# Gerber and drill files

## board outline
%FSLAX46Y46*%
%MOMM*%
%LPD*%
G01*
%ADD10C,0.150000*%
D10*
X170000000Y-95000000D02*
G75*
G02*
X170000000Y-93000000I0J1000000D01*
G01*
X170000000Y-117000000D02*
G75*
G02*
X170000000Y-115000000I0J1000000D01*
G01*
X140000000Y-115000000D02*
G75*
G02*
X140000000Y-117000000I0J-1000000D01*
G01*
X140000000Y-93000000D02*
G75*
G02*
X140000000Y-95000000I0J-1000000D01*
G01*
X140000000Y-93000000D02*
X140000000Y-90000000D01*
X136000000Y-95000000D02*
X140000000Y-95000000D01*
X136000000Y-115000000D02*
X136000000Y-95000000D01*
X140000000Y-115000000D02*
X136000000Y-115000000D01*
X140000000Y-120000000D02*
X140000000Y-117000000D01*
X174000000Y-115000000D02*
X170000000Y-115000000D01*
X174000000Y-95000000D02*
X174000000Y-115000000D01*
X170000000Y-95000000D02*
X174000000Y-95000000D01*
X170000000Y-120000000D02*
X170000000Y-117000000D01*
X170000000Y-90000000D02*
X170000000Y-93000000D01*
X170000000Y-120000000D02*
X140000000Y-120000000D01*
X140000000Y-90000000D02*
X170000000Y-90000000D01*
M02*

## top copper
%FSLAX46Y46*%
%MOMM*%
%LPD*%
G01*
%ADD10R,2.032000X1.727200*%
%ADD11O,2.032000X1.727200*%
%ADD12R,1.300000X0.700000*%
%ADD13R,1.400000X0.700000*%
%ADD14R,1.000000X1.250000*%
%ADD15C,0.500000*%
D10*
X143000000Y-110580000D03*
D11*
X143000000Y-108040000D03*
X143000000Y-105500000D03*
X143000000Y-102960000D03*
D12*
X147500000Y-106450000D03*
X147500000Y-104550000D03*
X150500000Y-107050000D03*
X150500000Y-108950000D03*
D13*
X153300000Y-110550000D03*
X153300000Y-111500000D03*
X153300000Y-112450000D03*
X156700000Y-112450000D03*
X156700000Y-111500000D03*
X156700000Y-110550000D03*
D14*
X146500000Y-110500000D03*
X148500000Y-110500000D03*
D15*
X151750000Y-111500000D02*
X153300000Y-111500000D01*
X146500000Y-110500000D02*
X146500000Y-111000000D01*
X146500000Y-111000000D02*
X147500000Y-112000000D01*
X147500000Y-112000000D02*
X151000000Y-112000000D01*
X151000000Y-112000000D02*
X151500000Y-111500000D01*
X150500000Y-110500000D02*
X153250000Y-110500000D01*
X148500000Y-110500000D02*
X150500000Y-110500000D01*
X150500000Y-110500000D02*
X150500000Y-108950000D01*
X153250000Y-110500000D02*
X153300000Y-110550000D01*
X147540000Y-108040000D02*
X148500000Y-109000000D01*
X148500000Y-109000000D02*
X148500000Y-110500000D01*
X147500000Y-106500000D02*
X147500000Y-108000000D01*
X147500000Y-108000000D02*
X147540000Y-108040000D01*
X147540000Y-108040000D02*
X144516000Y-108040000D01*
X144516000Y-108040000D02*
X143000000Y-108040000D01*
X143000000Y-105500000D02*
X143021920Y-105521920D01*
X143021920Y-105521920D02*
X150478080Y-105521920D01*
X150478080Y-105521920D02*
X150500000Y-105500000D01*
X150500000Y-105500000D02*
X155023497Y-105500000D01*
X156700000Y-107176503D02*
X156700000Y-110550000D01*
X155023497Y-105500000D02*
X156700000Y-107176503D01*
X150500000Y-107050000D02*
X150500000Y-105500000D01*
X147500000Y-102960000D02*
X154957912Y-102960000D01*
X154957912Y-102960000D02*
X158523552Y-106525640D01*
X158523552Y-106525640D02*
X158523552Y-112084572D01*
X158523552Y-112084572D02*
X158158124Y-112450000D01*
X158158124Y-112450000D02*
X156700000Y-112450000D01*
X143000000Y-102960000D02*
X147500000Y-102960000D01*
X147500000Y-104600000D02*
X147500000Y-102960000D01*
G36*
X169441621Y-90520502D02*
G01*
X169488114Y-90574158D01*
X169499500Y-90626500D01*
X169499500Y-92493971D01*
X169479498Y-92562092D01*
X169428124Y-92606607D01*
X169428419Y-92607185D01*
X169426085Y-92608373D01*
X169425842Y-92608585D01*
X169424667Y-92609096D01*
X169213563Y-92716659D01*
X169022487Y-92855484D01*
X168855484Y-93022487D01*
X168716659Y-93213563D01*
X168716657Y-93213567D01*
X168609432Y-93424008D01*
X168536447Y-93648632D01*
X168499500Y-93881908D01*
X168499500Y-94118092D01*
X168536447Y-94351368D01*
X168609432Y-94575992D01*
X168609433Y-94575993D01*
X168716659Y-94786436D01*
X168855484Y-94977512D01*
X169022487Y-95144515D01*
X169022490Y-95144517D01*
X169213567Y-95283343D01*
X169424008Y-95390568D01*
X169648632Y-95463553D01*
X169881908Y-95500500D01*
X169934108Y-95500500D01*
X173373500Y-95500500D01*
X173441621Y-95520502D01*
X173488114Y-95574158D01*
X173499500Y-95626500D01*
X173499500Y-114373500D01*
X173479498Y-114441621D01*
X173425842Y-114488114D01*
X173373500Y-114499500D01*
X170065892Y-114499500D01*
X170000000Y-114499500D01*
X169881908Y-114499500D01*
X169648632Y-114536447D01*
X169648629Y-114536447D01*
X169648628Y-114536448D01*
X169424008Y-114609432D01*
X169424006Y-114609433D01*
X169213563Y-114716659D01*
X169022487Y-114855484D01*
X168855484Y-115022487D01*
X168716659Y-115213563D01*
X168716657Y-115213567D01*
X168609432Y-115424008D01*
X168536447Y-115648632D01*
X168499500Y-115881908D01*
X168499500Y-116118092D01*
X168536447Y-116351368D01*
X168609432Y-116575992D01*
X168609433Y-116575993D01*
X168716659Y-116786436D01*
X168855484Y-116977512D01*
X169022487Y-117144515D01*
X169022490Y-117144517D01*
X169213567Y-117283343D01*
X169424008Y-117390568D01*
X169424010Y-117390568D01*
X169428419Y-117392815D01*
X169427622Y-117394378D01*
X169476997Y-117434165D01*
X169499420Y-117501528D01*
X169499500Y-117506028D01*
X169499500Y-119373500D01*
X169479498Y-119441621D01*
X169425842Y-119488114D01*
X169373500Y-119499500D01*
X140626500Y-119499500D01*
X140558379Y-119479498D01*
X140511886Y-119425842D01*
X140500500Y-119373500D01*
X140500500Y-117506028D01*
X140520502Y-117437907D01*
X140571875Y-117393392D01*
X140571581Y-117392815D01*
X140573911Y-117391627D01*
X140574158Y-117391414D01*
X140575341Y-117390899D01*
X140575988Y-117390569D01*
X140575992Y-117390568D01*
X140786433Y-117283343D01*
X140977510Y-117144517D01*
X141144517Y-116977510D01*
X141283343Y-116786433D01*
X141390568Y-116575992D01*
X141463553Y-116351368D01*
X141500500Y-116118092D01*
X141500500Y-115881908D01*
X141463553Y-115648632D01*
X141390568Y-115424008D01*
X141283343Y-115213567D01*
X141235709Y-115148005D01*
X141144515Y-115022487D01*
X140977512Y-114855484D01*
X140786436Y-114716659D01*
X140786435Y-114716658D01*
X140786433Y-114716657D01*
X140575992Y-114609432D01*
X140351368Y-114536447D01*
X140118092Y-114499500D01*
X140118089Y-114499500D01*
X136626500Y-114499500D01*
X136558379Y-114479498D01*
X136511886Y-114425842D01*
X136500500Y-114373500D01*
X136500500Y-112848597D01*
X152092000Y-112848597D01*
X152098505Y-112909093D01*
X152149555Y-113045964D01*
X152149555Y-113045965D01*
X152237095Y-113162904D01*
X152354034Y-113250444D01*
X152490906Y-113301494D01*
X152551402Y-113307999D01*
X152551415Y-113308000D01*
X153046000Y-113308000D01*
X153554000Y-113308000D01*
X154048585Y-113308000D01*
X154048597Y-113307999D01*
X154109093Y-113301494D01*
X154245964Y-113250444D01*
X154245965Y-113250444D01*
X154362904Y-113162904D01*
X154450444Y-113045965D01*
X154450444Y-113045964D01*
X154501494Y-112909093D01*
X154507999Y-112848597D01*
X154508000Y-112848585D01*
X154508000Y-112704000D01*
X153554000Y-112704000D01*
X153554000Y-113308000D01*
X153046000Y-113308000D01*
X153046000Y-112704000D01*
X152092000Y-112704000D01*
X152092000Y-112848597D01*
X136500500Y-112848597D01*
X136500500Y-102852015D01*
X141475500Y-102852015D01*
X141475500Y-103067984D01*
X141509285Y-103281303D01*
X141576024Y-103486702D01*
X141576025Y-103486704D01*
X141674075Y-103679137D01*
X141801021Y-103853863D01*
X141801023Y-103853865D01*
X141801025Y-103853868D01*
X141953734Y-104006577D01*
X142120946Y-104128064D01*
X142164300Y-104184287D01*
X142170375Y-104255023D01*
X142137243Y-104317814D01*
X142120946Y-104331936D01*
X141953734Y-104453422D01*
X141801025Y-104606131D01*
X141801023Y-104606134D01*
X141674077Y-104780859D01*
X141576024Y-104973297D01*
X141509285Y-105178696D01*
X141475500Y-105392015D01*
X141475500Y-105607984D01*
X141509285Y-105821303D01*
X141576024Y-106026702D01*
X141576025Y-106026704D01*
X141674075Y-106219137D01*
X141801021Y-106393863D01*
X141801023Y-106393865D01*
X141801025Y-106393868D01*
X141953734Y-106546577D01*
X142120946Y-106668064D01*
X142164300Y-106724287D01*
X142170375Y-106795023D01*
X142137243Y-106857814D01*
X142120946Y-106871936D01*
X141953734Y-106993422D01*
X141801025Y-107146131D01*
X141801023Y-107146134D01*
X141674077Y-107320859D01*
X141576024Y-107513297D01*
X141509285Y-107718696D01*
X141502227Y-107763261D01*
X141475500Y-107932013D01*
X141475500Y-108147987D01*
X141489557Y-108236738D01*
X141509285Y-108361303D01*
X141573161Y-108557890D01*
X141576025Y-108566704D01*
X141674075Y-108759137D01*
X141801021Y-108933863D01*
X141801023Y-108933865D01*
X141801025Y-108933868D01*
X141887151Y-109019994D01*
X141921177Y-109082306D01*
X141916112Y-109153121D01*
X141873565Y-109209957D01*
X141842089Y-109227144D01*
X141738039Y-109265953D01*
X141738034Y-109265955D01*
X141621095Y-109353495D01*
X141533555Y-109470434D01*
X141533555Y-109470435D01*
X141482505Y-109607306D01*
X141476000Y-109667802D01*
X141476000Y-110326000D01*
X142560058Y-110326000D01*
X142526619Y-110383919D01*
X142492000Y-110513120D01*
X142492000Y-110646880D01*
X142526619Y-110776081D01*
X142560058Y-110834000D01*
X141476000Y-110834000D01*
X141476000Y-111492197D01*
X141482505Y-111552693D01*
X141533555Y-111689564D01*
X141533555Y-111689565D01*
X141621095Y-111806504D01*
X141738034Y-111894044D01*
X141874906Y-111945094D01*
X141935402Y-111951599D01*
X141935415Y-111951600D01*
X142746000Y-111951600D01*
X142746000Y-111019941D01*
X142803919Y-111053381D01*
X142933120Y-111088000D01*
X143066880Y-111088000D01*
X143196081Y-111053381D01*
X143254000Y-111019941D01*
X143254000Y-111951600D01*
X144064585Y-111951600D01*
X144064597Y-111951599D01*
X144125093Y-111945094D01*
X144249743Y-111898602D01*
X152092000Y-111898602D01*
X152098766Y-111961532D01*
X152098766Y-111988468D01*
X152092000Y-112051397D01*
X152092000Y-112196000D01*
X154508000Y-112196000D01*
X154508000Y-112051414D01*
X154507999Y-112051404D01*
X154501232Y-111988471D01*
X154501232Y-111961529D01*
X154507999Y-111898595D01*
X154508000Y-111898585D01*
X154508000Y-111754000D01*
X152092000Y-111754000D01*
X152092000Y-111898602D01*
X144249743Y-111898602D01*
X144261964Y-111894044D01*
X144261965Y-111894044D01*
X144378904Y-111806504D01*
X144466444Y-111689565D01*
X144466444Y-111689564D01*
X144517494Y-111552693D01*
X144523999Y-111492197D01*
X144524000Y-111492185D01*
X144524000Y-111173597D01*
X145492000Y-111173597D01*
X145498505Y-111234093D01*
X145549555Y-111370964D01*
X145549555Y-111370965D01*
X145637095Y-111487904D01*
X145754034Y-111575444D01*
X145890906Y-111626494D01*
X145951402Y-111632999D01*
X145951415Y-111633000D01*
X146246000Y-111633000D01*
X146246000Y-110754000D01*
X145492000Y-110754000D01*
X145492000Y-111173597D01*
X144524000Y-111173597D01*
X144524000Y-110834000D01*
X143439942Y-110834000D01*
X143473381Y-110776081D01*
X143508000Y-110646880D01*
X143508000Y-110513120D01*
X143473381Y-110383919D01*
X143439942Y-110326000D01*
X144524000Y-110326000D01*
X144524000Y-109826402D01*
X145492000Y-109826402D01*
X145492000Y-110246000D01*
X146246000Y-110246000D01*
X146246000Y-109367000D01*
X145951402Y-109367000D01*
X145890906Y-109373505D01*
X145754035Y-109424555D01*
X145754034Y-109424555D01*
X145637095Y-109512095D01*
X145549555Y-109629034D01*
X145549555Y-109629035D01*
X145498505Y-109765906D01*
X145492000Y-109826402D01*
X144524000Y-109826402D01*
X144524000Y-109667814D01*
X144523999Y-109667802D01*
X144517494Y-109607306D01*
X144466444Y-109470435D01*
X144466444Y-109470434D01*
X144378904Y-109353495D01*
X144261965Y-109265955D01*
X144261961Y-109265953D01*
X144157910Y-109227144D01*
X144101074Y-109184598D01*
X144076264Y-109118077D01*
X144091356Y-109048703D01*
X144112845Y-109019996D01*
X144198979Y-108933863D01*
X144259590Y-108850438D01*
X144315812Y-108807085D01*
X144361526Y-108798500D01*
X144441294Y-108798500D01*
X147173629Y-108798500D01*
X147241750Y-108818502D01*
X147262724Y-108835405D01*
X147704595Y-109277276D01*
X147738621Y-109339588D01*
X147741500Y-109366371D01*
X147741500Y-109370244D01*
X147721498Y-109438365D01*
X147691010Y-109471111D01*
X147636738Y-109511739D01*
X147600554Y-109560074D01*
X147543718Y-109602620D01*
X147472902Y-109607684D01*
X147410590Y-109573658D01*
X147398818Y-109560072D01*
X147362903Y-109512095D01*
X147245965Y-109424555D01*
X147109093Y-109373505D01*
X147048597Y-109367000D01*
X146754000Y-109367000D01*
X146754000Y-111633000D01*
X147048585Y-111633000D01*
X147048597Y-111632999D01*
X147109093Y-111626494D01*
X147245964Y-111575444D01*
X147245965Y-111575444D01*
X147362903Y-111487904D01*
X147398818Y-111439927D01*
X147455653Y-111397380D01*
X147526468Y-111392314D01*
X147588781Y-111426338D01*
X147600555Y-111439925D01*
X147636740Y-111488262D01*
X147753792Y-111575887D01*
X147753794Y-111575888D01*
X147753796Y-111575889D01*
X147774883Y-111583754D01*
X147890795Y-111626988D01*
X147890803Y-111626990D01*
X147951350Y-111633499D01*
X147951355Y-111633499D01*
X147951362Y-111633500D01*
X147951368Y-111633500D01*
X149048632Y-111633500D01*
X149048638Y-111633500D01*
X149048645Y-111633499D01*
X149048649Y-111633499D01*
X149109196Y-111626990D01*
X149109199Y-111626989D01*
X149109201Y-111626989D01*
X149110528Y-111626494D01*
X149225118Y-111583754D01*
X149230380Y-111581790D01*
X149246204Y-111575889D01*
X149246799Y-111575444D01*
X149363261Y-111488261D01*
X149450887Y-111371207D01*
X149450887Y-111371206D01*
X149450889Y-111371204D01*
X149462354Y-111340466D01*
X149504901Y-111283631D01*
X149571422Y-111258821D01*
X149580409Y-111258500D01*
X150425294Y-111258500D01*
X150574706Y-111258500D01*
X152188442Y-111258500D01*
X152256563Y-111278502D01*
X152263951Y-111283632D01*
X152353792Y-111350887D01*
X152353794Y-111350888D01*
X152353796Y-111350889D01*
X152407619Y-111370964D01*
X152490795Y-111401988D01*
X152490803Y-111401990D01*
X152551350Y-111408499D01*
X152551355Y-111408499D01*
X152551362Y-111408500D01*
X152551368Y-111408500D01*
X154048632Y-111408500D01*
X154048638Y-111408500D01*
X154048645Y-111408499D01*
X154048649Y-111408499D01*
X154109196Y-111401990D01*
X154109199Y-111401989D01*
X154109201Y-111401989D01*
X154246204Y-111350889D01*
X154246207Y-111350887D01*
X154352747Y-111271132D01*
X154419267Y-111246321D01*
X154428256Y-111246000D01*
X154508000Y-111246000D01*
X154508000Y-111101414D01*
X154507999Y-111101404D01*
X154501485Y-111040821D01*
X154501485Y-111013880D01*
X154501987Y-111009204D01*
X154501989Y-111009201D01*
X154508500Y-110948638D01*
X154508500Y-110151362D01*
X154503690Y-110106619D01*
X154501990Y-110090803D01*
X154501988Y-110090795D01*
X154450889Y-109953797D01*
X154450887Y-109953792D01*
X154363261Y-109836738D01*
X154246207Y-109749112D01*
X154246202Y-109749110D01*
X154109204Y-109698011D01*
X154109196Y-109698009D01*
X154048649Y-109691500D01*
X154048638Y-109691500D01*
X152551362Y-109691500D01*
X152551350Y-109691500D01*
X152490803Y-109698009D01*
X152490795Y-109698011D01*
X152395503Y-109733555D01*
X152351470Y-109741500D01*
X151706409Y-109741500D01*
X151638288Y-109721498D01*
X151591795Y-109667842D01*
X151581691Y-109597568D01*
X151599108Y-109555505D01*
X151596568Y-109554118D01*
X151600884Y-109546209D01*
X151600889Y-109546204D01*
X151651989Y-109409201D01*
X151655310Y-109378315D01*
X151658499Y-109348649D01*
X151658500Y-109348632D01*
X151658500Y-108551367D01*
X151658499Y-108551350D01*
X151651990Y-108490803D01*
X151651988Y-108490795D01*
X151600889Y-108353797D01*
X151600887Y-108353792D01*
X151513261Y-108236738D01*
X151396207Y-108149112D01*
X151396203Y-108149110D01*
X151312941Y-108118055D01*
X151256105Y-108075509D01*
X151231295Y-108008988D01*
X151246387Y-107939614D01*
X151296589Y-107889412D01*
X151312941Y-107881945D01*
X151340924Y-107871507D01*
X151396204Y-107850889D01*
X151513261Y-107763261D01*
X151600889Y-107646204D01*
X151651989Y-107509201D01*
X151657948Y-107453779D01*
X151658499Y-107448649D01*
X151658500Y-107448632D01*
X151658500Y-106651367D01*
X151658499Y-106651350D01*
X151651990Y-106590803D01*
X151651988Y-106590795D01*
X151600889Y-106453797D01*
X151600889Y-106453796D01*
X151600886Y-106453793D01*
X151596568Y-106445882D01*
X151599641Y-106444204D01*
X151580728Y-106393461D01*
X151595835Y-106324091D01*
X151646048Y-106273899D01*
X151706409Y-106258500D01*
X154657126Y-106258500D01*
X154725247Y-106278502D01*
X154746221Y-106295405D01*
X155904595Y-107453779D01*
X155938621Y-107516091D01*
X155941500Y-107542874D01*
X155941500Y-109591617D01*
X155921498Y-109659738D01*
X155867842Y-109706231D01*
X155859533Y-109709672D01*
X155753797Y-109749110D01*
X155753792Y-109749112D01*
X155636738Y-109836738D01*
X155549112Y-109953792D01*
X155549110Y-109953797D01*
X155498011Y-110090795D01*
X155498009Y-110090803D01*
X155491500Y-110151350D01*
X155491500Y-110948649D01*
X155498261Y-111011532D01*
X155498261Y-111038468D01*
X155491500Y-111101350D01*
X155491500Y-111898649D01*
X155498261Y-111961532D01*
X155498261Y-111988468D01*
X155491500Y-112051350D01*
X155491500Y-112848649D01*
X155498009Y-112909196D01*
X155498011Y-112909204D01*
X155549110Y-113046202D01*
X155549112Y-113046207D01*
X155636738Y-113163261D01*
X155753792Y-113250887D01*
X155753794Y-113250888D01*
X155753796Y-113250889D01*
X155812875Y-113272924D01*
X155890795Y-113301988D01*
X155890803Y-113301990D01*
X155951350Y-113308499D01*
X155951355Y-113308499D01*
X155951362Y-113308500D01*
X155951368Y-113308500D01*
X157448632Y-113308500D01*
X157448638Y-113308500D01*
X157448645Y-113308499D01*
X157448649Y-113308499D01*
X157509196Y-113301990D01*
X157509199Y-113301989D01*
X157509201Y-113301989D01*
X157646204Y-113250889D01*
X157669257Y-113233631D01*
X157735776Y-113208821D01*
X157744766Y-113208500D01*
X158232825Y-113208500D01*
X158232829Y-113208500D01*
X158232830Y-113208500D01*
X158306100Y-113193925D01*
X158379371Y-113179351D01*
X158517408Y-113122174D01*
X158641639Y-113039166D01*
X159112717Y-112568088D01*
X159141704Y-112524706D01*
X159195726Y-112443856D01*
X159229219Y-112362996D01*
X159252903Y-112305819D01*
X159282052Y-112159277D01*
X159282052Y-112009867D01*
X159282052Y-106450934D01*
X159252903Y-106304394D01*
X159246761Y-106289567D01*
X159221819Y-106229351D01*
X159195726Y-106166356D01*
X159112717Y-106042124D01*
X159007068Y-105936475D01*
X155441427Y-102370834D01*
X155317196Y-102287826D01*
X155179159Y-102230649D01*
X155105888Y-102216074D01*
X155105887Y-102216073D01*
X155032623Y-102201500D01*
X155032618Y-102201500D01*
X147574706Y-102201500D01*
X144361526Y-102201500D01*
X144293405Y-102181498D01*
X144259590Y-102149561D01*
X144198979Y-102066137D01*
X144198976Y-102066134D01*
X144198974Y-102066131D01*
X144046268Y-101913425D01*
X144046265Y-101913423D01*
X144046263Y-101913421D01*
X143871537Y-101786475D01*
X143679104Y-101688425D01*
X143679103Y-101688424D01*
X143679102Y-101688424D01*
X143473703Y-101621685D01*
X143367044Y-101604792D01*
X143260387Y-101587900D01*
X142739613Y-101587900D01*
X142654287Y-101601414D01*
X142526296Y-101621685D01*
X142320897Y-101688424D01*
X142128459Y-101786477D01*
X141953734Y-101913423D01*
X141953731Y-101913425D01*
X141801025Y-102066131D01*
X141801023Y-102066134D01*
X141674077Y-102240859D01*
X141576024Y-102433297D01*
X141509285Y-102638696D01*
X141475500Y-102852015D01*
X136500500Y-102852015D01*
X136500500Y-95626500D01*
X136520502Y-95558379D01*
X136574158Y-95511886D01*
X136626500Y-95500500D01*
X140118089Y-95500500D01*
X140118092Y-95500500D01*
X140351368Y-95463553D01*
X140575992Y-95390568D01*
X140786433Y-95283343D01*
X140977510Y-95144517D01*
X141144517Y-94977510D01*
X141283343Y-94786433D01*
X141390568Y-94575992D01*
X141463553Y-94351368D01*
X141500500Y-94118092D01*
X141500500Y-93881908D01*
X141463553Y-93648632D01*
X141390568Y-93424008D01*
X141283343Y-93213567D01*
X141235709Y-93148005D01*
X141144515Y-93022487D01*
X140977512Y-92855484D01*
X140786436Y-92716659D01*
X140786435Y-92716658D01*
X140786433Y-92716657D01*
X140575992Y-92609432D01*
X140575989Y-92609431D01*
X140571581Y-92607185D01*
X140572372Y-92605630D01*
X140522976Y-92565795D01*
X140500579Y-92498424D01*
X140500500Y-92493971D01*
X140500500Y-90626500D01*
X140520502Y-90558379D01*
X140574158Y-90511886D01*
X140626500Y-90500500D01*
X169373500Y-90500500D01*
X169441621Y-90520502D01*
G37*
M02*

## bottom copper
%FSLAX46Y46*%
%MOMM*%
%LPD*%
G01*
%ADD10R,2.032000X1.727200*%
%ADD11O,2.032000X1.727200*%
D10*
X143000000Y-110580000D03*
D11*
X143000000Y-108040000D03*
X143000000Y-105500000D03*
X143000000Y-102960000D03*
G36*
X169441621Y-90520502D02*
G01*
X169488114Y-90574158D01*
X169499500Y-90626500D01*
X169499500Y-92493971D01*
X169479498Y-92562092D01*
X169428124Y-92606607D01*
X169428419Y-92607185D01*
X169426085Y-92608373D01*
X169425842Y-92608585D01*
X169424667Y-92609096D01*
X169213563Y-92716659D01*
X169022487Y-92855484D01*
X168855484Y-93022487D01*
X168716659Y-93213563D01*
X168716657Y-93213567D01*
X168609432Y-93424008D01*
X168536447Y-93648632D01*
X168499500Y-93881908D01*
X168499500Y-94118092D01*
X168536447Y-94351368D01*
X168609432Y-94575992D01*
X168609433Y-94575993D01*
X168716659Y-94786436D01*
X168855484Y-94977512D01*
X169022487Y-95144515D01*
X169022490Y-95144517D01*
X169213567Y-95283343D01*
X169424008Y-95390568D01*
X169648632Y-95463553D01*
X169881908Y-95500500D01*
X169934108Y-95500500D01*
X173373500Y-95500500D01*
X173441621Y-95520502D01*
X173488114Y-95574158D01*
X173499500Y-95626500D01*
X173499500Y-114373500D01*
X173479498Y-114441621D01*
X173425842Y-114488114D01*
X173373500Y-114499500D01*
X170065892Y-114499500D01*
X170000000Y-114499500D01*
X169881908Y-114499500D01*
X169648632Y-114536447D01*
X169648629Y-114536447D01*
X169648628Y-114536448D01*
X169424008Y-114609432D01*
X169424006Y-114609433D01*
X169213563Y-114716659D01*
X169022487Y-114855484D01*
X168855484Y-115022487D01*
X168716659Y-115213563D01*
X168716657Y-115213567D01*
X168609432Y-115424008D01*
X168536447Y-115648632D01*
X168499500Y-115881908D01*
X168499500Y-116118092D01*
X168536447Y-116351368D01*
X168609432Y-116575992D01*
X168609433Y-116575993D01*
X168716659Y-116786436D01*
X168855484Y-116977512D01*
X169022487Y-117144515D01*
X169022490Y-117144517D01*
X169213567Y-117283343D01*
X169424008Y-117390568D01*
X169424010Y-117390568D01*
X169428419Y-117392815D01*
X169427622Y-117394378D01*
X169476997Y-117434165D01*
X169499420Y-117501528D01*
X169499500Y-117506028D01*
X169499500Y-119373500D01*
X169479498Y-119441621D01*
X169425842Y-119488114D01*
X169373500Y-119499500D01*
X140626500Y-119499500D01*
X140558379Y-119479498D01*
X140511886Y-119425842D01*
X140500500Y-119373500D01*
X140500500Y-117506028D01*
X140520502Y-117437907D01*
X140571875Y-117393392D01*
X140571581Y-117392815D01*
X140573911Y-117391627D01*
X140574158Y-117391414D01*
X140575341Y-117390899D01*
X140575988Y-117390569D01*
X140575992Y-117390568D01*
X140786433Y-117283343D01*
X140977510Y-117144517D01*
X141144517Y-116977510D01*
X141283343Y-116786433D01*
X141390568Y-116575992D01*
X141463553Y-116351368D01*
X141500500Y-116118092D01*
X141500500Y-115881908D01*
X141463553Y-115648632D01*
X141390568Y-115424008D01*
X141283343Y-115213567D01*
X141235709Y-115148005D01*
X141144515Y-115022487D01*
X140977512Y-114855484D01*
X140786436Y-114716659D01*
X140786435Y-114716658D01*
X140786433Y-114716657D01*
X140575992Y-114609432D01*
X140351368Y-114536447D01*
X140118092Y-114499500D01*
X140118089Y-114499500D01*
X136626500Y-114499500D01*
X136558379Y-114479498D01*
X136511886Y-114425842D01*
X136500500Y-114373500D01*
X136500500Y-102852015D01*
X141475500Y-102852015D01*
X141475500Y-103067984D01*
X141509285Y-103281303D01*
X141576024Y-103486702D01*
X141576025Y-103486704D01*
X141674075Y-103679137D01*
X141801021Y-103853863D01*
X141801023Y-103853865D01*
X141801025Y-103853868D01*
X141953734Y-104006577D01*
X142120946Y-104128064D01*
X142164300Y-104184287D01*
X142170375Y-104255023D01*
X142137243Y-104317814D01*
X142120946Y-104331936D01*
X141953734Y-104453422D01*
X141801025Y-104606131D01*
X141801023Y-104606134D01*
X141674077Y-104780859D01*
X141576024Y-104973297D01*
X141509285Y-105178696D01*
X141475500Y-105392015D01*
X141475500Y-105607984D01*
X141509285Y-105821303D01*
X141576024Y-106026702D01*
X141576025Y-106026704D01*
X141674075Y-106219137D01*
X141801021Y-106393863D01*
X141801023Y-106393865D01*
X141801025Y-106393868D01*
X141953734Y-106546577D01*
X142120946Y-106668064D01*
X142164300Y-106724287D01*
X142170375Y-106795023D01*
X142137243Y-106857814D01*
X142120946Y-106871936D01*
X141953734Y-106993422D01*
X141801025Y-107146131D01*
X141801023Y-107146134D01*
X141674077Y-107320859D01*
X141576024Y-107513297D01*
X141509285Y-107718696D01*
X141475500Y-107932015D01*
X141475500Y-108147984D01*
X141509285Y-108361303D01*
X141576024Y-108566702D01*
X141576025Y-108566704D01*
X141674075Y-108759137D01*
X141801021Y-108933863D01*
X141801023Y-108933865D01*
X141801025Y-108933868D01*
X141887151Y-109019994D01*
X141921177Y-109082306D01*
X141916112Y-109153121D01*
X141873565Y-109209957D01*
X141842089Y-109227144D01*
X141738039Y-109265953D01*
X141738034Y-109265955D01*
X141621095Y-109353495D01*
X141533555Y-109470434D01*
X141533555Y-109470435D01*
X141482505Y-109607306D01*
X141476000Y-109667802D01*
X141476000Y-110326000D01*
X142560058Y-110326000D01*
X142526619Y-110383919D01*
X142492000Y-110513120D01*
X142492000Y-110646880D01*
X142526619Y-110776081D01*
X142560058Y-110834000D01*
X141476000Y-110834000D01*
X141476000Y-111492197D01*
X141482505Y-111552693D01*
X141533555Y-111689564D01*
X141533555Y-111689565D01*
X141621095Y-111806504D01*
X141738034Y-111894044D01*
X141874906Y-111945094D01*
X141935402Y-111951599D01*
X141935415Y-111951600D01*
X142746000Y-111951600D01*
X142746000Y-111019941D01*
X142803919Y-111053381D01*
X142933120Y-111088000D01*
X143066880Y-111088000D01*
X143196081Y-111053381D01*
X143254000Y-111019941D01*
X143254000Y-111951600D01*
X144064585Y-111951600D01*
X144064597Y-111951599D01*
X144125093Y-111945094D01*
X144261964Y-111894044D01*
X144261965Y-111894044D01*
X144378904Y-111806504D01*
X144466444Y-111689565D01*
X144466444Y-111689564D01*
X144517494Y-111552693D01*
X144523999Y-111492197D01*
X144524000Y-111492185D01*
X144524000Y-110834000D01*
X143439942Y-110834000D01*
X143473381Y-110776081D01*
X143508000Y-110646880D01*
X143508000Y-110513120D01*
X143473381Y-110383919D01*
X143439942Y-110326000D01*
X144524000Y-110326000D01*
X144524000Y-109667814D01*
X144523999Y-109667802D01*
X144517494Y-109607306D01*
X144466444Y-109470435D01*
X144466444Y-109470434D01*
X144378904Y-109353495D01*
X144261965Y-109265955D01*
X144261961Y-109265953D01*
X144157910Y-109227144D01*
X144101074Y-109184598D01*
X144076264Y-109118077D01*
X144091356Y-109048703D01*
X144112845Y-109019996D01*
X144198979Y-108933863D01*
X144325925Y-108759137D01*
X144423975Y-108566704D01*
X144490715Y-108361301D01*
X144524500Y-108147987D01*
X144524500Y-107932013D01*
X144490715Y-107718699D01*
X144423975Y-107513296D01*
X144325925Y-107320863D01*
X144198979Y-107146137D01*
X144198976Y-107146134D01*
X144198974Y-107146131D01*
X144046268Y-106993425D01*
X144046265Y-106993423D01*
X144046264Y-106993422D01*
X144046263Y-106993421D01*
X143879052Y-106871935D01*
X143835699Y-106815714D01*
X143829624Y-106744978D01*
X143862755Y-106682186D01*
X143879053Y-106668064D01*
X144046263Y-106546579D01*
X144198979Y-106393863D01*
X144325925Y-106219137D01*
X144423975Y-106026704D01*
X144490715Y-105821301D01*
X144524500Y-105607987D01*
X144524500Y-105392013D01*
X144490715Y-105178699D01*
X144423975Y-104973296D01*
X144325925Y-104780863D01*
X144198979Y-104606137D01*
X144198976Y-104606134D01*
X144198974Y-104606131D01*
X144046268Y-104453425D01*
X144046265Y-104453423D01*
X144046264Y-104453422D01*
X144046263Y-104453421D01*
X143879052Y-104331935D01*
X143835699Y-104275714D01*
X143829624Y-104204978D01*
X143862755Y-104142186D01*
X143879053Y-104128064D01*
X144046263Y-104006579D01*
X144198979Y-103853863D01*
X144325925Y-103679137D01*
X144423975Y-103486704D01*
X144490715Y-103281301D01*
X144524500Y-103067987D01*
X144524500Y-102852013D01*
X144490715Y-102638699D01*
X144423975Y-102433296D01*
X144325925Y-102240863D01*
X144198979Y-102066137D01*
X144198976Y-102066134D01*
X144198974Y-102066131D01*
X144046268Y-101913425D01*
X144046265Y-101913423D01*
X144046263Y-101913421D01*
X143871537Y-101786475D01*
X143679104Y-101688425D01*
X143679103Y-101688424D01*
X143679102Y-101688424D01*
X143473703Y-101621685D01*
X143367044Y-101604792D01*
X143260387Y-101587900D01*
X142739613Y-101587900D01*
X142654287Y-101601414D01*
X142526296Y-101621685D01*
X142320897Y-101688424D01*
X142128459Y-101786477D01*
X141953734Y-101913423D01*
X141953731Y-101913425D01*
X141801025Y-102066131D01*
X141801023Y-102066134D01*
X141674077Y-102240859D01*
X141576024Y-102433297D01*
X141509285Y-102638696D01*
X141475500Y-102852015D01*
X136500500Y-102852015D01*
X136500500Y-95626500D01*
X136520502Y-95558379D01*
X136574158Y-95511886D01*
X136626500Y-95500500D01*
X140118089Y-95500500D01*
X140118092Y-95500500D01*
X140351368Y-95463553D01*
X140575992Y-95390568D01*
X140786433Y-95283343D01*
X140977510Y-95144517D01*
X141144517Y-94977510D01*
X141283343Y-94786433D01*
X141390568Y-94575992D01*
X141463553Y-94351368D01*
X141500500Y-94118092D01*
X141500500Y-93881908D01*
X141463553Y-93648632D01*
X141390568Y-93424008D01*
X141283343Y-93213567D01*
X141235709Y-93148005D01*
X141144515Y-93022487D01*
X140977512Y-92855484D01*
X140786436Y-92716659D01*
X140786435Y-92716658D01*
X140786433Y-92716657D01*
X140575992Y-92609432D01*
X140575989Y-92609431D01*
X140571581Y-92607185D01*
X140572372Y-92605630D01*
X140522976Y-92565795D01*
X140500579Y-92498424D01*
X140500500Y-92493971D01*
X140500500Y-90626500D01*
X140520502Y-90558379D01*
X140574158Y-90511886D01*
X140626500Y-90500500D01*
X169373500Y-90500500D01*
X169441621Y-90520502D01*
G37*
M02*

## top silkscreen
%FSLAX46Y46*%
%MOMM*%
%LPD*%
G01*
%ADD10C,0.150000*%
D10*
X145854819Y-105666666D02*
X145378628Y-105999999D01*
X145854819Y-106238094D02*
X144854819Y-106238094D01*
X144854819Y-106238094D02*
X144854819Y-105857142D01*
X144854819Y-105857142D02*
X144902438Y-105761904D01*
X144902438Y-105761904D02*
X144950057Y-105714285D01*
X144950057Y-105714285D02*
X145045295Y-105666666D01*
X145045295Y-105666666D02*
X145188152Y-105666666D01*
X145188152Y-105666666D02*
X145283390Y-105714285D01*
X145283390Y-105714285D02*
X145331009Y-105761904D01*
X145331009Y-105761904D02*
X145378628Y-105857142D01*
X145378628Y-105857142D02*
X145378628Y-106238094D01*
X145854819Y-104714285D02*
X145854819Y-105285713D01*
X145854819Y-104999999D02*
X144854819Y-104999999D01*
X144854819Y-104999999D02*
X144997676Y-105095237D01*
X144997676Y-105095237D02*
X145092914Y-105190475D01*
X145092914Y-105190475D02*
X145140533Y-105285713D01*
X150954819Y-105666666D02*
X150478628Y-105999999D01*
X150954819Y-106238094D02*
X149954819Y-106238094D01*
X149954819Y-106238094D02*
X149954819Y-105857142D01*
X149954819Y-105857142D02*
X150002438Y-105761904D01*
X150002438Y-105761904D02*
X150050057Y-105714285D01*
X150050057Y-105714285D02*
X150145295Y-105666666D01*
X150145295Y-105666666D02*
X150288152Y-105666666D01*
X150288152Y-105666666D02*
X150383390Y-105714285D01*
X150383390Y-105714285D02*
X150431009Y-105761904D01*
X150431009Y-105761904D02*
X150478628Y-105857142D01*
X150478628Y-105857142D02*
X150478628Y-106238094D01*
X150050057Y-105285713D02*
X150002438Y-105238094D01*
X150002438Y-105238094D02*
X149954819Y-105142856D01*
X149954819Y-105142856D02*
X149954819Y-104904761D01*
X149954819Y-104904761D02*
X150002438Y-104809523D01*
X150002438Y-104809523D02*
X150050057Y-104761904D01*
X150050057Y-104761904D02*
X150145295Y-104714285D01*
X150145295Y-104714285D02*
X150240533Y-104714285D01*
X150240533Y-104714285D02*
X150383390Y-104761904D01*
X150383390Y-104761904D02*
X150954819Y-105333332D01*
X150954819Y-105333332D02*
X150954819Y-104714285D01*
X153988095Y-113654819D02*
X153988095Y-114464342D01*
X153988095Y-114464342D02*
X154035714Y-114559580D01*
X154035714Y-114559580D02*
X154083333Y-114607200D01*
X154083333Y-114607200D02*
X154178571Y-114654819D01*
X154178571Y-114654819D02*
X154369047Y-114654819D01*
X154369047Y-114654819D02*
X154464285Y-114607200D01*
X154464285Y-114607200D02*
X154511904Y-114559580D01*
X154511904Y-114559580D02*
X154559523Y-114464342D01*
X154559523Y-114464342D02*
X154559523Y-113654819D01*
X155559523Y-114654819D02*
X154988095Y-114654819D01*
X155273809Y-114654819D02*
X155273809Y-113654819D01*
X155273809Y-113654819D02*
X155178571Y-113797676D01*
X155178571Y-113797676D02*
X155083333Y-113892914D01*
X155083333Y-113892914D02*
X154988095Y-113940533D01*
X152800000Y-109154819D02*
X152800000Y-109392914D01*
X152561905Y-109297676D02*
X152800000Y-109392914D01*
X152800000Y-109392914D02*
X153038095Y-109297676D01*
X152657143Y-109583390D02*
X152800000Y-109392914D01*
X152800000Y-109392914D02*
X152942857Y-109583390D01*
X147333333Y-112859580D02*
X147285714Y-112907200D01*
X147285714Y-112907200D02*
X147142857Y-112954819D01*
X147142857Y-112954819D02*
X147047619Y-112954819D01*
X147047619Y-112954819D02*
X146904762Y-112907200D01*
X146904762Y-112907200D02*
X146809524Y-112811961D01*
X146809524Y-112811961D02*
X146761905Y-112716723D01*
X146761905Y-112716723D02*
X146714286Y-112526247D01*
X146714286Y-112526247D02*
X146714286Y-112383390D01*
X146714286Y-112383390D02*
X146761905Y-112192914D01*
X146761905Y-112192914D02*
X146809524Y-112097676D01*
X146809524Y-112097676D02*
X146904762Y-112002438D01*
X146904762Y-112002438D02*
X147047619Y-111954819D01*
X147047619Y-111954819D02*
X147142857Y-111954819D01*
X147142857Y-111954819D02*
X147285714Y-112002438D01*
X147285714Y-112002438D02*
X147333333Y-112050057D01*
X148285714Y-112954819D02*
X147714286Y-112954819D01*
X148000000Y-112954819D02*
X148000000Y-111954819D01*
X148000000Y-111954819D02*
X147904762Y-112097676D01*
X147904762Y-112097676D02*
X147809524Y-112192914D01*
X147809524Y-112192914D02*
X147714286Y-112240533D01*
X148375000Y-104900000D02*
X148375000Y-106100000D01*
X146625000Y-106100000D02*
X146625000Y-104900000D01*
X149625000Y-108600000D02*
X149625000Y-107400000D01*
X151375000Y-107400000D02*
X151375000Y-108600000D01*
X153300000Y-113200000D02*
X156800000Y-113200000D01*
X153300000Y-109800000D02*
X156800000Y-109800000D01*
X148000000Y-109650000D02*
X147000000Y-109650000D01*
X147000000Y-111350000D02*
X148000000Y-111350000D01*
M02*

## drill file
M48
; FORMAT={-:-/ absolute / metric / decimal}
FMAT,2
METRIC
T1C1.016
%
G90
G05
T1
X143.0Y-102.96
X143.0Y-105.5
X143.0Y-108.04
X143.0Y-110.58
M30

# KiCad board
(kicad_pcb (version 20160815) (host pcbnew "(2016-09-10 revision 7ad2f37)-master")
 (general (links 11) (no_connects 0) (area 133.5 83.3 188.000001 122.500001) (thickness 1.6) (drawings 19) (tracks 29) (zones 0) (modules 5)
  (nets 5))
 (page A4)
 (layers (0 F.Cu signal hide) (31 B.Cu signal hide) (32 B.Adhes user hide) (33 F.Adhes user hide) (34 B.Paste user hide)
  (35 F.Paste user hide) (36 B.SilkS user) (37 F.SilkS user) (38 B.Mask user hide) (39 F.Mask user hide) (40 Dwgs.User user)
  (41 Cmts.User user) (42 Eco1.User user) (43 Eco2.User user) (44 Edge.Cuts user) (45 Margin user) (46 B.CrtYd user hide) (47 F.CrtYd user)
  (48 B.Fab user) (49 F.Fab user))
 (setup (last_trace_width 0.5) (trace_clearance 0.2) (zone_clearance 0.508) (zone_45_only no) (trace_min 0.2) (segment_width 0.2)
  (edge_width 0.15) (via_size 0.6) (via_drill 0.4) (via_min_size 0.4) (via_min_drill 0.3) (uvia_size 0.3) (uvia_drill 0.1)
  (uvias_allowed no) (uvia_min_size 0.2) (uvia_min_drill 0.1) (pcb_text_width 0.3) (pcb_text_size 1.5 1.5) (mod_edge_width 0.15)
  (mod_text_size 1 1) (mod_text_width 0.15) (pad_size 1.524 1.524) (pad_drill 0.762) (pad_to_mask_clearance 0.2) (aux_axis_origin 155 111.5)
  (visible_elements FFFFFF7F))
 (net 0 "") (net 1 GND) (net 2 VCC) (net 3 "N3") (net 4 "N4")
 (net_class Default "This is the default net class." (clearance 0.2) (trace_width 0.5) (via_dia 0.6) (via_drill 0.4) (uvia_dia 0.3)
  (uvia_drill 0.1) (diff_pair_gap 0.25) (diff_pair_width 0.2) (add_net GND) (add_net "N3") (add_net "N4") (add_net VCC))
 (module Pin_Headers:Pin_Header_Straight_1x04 (layer B.Cu) (at 143 110.58)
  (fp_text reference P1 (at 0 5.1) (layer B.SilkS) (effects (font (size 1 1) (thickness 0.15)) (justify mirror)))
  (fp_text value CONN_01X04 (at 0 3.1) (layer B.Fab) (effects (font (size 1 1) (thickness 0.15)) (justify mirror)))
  (pad 1 thru_hole rect (at 0 0) (size 2.032 1.7272) (drill 1.016) (layers *.Cu *.Mask B.SilkS) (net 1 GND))
  (pad 2 thru_hole oval (at 0 -2.54) (size 2.032 1.7272) (drill 1.016) (layers *.Cu *.Mask B.SilkS) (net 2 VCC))
  (pad 3 thru_hole oval (at 0 -5.08) (size 2.032 1.7272) (drill 1.016) (layers *.Cu *.Mask B.SilkS) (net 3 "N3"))
  (pad 4 thru_hole oval (at 0 -7.62) (size 2.032 1.7272) (drill 1.016) (layers *.Cu *.Mask B.SilkS) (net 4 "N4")))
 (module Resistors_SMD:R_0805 (layer F.Cu) (at 147.5 105.5 90)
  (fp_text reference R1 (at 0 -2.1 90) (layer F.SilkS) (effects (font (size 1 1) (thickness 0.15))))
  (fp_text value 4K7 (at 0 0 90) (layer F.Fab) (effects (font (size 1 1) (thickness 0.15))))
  (fp_line (start 0.6 0.875) (end -0.6 0.875) (layer F.SilkS) (width 0.15))
  (fp_line (start -0.6 -0.875) (end 0.6 -0.875) (layer F.SilkS) (width 0.15))
  (pad 1 smd rect (at -0.95 0 90) (size 0.7 1.3) (layers F.Cu F.Paste F.Mask) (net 2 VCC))
  (pad 2 smd rect (at 0.95 0 90) (size 0.7 1.3) (layers F.Cu F.Paste F.Mask) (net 4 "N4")))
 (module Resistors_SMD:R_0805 (layer F.Cu) (at 150.5 108 270)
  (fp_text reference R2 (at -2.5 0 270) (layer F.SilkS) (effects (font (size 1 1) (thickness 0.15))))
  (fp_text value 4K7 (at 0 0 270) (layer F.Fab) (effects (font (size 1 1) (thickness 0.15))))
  (fp_line (start 0.6 0.875) (end -0.6 0.875) (layer F.SilkS) (width 0.15))
  (fp_line (start -0.6 -0.875) (end 0.6 -0.875) (layer F.SilkS) (width 0.15))
  (pad 1 smd rect (at -0.95 0 270) (size 0.7 1.3) (layers F.Cu F.Paste F.Mask) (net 3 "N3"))
  (pad 2 smd rect (at 0.95 0 270) (size 0.7 1.3) (layers F.Cu F.Paste F.Mask) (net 2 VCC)))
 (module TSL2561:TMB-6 (layer F.Cu) (at 155 111.5)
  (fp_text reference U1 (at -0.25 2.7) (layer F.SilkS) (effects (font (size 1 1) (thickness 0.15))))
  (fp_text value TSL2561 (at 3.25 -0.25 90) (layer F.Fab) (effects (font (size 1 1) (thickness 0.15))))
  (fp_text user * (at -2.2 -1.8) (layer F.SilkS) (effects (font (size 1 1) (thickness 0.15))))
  (fp_line (start -1.7 1.7) (end 1.8 1.7) (layer F.SilkS) (width 0.15))
  (fp_line (start -1.7 -1.7) (end 1.8 -1.7) (layer F.SilkS) (width 0.15))
  (pad 1 smd rect (at -1.7 -0.95) (size 1.4 0.7) (layers F.Cu F.Paste F.Mask) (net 2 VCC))
  (pad 2 smd rect (at -1.7 0) (size 1.4 0.7) (layers F.Cu F.Paste F.Mask) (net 1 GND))
  (pad 3 smd rect (at -1.7 0.95) (size 1.4 0.7) (layers F.Cu F.Paste F.Mask) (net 1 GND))
  (pad 4 smd rect (at 1.7 0.95) (size 1.4 0.7) (layers F.Cu F.Paste F.Mask) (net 4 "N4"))
  (pad 5 smd rect (at 1.7 0) (size 1.4 0.7) (layers F.Cu F.Paste F.Mask))
  (pad 6 smd rect (at 1.7 -0.95) (size 1.4 0.7) (layers F.Cu F.Paste F.Mask) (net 3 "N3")))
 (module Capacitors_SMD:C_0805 (layer F.Cu) (at 147.5 110.5)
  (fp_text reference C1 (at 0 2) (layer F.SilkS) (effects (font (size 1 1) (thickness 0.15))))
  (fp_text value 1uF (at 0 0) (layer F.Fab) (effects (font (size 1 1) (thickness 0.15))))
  (fp_line (start 0.5 -0.85) (end -0.5 -0.85) (layer F.SilkS) (width 0.15))
  (fp_line (start -0.5 0.85) (end 0.5 0.85) (layer F.SilkS) (width 0.15))
  (pad 1 smd rect (at -1 0) (size 1 1.25) (layers F.Cu F.Paste F.Mask) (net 1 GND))
  (pad 2 smd rect (at 1 0) (size 1 1.25) (layers F.Cu F.Paste F.Mask) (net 2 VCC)))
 (gr_arc (start 170 94) (end 170 95) (angle 180) (layer Edge.Cuts) (width 0.15))
 (gr_arc (start 170 116) (end 170 117) (angle 180) (layer Edge.Cuts) (width 0.15))
 (gr_arc (start 140 116) (end 140 115) (angle 180) (layer Edge.Cuts) (width 0.15))
 (gr_arc (start 140 94) (end 140 93) (angle 180) (layer Edge.Cuts) (width 0.15))
 (gr_line (start 140 93) (end 140 90) (layer Edge.Cuts) (width 0.15))
 (gr_line (start 136 95) (end 140 95) (layer Edge.Cuts) (width 0.15))
 (gr_line (start 136 115) (end 136 95) (layer Edge.Cuts) (width 0.15))
 (gr_line (start 140 115) (end 136 115) (layer Edge.Cuts) (width 0.15))
 (gr_line (start 140 120) (end 140 117) (layer Edge.Cuts) (width 0.15))
 (gr_line (start 174 115) (end 170 115) (layer Edge.Cuts) (width 0.15))
 (gr_line (start 174 95) (end 174 115) (layer Edge.Cuts) (width 0.15))
 (gr_line (start 170 95) (end 174 95) (layer Edge.Cuts) (width 0.15))
 (gr_line (start 170 120) (end 170 117) (layer Edge.Cuts) (width 0.15))
 (gr_line (start 170 90) (end 170 93) (layer Edge.Cuts) (width 0.15))
 (gr_line (start 170 120) (end 140 120) (layer Edge.Cuts) (width 0.15))
 (gr_line (start 140 90) (end 170 90) (layer Edge.Cuts) (width 0.15))
 (segment (start 151.75 111.5) (end 153.3 111.5) (width 0.5) (layer F.Cu) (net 1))
 (segment (start 146.5 110.5) (end 146.5 111) (width 0.5) (layer F.Cu) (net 1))
 (segment (start 146.5 111) (end 147.5 112) (width 0.5) (layer F.Cu) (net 1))
 (segment (start 147.5 112) (end 151 112) (width 0.5) (layer F.Cu) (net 1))
 (segment (start 151 112) (end 151.5 111.5) (width 0.5) (layer F.Cu) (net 1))
 (segment (start 150.5 110.5) (end 153.25 110.5) (width 0.5) (layer F.Cu) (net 2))
 (segment (start 148.5 110.5) (end 150.5 110.5) (width 0.5) (layer F.Cu) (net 2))
 (segment (start 150.5 110.5) (end 150.5 108.95) (width 0.5) (layer F.Cu) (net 2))
 (segment (start 153.25 110.5) (end 153.3 110.55) (width 0.5) (layer F.Cu) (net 2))
 (segment (start 147.54 108.04) (end 148.5 109) (width 0.5) (layer F.Cu) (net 2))
 (segment (start 148.5 109) (end 148.5 110.5) (width 0.5) (layer F.Cu) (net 2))
 (segment (start 147.5 106.5) (end 147.5 108) (width 0.5) (layer F.Cu) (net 2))
 (segment (start 147.5 108) (end 147.54 108.04) (width 0.5) (layer F.Cu) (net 2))
 (segment (start 147.54 108.04) (end 144.516 108.04) (width 0.5) (layer F.Cu) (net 2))
 (segment (start 144.516 108.04) (end 143 108.04) (width 0.5) (layer F.Cu) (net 2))
 (segment (start 143 105.5) (end 143.02192 105.52192) (width 0.5) (layer F.Cu) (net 3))
 (segment (start 143.02192 105.52192) (end 150.47808 105.52192) (width 0.5) (layer F.Cu) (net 3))
 (segment (start 150.47808 105.52192) (end 150.5 105.5) (width 0.5) (layer F.Cu) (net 3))
 (segment (start 150.5 105.5) (end 155.023497 105.5) (width 0.5) (layer F.Cu) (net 3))
 (segment (start 156.7 107.176503) (end 156.7 110.55) (width 0.5) (layer F.Cu) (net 3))
 (segment (start 155.023497 105.5) (end 156.7 107.176503) (width 0.5) (layer F.Cu) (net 3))
 (segment (start 150.5 107.05) (end 150.5 105.5) (width 0.5) (layer F.Cu) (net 3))
 (segment (start 147.5 102.96) (end 154.957912 102.96) (width 0.5) (layer F.Cu) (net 4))
 (segment (start 154.957912 102.96) (end 158.523552 106.52564) (width 0.5) (layer F.Cu) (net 4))
 (segment (start 158.523552 106.52564) (end 158.523552 112.084572) (width 0.5) (layer F.Cu) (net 4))
 (segment (start 158.523552 112.084572) (end 158.158124 112.45) (width 0.5) (layer F.Cu) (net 4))
 (segment (start 158.158124 112.45) (end 156.7 112.45) (width 0.5) (layer F.Cu) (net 4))
 (segment (start 143 102.96) (end 147.5 102.96) (width 0.5) (layer F.Cu) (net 4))
 (segment (start 147.5 104.6) (end 147.5 102.96) (width 0.5) (layer F.Cu) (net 4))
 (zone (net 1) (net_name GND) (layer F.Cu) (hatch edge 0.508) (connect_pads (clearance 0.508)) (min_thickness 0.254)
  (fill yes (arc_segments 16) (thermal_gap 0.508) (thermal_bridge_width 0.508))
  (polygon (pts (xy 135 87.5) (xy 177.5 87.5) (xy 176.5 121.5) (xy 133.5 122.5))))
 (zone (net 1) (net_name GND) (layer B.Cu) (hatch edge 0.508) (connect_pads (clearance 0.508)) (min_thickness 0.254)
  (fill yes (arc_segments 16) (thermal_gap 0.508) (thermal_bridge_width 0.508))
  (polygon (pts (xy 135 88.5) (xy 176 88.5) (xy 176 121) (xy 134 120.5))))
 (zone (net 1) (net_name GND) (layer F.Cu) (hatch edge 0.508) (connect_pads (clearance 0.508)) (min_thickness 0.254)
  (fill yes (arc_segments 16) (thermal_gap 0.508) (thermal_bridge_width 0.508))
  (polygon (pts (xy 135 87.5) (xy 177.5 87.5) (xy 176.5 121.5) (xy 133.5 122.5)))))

